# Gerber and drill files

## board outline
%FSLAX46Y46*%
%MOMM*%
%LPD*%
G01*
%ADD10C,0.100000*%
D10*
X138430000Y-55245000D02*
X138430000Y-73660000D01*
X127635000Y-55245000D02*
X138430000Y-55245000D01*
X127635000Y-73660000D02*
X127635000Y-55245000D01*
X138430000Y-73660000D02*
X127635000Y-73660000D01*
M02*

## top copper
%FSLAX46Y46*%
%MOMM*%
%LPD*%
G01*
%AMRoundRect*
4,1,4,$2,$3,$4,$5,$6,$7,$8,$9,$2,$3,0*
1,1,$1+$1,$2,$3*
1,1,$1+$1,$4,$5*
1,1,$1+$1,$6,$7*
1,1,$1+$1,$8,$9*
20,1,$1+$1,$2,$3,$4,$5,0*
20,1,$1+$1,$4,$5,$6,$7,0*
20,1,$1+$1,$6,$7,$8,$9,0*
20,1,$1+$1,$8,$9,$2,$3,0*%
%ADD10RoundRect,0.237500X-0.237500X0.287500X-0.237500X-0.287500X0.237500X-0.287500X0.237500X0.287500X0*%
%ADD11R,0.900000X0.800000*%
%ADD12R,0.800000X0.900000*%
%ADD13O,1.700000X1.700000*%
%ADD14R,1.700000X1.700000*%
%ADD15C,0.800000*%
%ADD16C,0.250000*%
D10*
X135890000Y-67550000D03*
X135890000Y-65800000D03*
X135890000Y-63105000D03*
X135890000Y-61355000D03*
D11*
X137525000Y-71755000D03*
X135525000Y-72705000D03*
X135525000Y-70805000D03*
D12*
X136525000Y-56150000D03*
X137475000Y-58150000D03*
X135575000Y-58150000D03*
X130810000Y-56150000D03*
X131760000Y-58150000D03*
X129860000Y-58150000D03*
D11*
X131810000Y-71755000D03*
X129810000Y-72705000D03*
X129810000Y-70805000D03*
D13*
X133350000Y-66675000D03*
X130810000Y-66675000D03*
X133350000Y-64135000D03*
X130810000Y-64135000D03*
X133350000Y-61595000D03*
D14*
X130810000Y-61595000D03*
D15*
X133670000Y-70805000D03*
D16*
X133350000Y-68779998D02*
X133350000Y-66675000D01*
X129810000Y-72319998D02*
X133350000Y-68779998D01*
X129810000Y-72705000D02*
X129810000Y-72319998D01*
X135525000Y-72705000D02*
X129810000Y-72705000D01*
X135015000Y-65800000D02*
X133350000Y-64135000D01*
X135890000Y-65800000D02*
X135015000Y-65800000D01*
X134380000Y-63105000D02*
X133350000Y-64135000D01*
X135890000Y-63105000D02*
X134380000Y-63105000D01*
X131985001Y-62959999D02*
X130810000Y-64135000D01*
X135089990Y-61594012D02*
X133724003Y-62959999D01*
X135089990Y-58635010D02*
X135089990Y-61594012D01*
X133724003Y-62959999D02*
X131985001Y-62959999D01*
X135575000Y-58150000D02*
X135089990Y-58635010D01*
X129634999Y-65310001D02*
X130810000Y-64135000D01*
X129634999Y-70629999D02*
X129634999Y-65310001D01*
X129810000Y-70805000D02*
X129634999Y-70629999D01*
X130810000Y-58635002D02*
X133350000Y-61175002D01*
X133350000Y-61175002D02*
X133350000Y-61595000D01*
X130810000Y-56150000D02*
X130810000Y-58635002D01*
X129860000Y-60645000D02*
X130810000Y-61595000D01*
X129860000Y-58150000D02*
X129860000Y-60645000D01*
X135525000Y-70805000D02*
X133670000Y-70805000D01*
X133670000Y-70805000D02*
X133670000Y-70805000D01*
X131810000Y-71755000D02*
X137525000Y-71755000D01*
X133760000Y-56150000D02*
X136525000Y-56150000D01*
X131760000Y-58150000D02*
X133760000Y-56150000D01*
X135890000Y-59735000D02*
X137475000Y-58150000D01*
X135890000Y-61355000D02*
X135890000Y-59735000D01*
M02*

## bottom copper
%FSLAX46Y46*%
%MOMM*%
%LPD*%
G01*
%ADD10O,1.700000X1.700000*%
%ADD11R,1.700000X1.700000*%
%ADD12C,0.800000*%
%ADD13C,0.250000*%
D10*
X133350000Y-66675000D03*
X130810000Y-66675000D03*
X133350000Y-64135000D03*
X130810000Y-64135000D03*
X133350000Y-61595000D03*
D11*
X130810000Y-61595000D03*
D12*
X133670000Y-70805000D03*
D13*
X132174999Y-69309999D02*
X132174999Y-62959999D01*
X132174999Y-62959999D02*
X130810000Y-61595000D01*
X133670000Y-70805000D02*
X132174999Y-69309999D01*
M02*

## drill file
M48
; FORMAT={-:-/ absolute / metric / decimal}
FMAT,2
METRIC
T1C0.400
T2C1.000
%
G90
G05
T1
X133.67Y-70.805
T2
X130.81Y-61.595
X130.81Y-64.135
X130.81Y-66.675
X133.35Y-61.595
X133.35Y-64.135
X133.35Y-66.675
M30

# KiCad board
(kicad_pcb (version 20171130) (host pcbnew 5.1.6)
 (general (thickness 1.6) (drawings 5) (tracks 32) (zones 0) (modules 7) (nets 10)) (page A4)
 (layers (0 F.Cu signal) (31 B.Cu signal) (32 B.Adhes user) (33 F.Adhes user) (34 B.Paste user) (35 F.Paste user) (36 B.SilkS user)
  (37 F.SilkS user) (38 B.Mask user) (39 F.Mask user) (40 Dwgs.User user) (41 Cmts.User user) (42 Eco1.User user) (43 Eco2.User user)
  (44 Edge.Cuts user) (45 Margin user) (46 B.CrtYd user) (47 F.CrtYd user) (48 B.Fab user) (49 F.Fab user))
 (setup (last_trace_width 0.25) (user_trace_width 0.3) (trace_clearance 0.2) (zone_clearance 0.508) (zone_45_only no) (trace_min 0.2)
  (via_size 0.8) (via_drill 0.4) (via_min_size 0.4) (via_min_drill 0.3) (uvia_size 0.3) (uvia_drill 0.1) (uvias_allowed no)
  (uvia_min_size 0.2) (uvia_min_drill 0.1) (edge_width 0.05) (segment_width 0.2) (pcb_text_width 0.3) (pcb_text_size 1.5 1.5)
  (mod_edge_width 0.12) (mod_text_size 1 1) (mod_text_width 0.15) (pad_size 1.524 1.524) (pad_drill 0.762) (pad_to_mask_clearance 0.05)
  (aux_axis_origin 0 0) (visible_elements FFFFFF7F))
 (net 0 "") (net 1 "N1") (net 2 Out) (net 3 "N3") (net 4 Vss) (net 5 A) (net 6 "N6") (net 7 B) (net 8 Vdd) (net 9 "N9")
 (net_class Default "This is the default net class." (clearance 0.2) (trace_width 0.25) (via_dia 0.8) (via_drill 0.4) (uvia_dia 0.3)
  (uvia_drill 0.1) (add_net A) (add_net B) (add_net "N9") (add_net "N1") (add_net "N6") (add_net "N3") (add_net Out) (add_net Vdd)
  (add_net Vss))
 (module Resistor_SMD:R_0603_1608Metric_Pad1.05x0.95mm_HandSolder (layer F.Cu) (at 135.89 66.675 270)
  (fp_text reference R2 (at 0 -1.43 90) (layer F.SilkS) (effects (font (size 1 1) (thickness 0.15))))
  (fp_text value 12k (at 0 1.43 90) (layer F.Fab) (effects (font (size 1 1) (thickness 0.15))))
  (pad 2 smd roundrect (at 0.875 0 270) (size 1.05 0.95) (layers F.Cu F.Paste F.Mask) (roundrect_rratio 0.25) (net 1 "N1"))
  (pad 1 smd roundrect (at -0.875 0 270) (size 1.05 0.95) (layers F.Cu F.Paste F.Mask) (roundrect_rratio 0.25) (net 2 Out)))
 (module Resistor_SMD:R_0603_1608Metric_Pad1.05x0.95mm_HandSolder (layer F.Cu) (at 135.89 62.23 270)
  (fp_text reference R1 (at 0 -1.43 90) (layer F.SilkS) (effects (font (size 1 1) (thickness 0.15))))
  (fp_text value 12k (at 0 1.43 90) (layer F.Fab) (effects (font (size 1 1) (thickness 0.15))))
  (pad 2 smd roundrect (at 0.875 0 270) (size 1.05 0.95) (layers F.Cu F.Paste F.Mask) (roundrect_rratio 0.25) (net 2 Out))
  (pad 1 smd roundrect (at -0.875 0 270) (size 1.05 0.95) (layers F.Cu F.Paste F.Mask) (roundrect_rratio 0.25) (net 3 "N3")))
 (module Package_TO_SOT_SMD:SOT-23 (layer F.Cu) (at 136.525 71.755)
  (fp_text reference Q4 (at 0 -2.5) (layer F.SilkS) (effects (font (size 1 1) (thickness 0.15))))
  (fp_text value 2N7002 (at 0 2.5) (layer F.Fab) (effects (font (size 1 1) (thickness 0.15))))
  (pad 3 smd rect (at 1 0) (size 0.9 0.8) (layers F.Cu F.Paste F.Mask) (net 1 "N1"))
  (pad 2 smd rect (at -1 0.95) (size 0.9 0.8) (layers F.Cu F.Paste F.Mask) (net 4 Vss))
  (pad 1 smd rect (at -1 -0.95) (size 0.9 0.8) (layers F.Cu F.Paste F.Mask) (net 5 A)))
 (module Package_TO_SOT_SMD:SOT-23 (layer F.Cu) (at 136.525 57.15 90)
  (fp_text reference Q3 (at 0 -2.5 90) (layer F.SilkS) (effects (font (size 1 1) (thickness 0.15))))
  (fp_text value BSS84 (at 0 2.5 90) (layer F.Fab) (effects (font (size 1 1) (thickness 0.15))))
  (pad 3 smd rect (at 1 0 90) (size 0.9 0.8) (layers F.Cu F.Paste F.Mask) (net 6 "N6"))
  (pad 2 smd rect (at -1 0.95 90) (size 0.9 0.8) (layers F.Cu F.Paste F.Mask) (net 3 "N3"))
  (pad 1 smd rect (at -1 -0.95 90) (size 0.9 0.8) (layers F.Cu F.Paste F.Mask) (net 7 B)))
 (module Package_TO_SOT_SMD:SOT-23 (layer F.Cu) (at 130.81 57.15 90)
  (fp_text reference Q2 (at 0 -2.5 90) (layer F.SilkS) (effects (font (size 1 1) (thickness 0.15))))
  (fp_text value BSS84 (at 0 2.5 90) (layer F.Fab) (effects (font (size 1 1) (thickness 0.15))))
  (pad 3 smd rect (at 1 0 90) (size 0.9 0.8) (layers F.Cu F.Paste F.Mask) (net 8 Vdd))
  (pad 2 smd rect (at -1 0.95 90) (size 0.9 0.8) (layers F.Cu F.Paste F.Mask) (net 6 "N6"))
  (pad 1 smd rect (at -1 -0.95 90) (size 0.9 0.8) (layers F.Cu F.Paste F.Mask) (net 5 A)))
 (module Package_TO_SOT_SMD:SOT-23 (layer F.Cu) (at 130.81 71.755)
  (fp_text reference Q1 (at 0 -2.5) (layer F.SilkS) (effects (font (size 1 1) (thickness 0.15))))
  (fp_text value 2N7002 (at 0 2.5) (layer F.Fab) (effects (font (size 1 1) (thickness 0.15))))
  (pad 3 smd rect (at 1 0) (size 0.9 0.8) (layers F.Cu F.Paste F.Mask) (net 1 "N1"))
  (pad 2 smd rect (at -1 0.95) (size 0.9 0.8) (layers F.Cu F.Paste F.Mask) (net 4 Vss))
  (pad 1 smd rect (at -1 -0.95) (size 0.9 0.8) (layers F.Cu F.Paste F.Mask) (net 7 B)))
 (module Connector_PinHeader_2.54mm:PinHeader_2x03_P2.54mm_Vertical (layer F.Cu) (at 130.81 61.595)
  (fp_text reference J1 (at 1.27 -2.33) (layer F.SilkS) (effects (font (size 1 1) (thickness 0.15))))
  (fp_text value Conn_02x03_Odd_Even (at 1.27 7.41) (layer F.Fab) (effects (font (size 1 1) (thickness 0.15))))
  (pad 6 thru_hole oval (at 2.54 5.08) (size 1.7 1.7) (drill 1) (layers *.Cu *.Mask) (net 4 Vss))
  (pad 5 thru_hole oval (at 0 5.08) (size 1.7 1.7) (drill 1) (layers *.Cu *.Mask) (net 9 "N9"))
  (pad 4 thru_hole oval (at 2.54 2.54) (size 1.7 1.7) (drill 1) (layers *.Cu *.Mask) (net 2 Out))
  (pad 3 thru_hole oval (at 0 2.54) (size 1.7 1.7) (drill 1) (layers *.Cu *.Mask) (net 7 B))
  (pad 2 thru_hole oval (at 2.54 0) (size 1.7 1.7) (drill 1) (layers *.Cu *.Mask) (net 8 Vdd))
  (pad 1 thru_hole rect (at 0 0) (size 1.7 1.7) (drill 1) (layers *.Cu *.Mask) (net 5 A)))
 (gr_line (start 138.43 55.245) (end 138.43 73.66) (layer Edge.Cuts) (width 0.1))
 (gr_line (start 127.635 55.245) (end 138.43 55.245) (layer Edge.Cuts) (width 0.1))
 (gr_line (start 127.635 73.66) (end 127.635 55.245) (layer Edge.Cuts) (width 0.1))
 (gr_line (start 138.43 73.66) (end 127.635 73.66) (layer Edge.Cuts) (width 0.1))
 (segment (start 133.35 68.779998) (end 133.35 66.675) (width 0.25) (layer F.Cu) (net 4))
 (segment (start 129.81 72.319998) (end 133.35 68.779998) (width 0.25) (layer F.Cu) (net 4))
 (segment (start 129.81 72.705) (end 129.81 72.319998) (width 0.25) (layer F.Cu) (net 4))
 (segment (start 135.525 72.705) (end 129.81 72.705) (width 0.25) (layer F.Cu) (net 4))
 (segment (start 135.015 65.8) (end 133.35 64.135) (width 0.25) (layer F.Cu) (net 2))
 (segment (start 135.89 65.8) (end 135.015 65.8) (width 0.25) (layer F.Cu) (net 2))
 (segment (start 134.38 63.105) (end 133.35 64.135) (width 0.25) (layer F.Cu) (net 2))
 (segment (start 135.89 63.105) (end 134.38 63.105) (width 0.25) (layer F.Cu) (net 2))
 (segment (start 131.985001 62.959999) (end 130.81 64.135) (width 0.25) (layer F.Cu) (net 7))
 (segment (start 135.08999 61.594012) (end 133.724003 62.959999) (width 0.25) (layer F.Cu) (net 7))
 (segment (start 135.08999 58.63501) (end 135.08999 61.594012) (width 0.25) (layer F.Cu) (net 7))
 (segment (start 133.724003 62.959999) (end 131.985001 62.959999) (width 0.25) (layer F.Cu) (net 7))
 (segment (start 135.575 58.15) (end 135.08999 58.63501) (width 0.25) (layer F.Cu) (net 7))
 (segment (start 129.634999 65.310001) (end 130.81 64.135) (width 0.25) (layer F.Cu) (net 7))
 (segment (start 129.634999 70.629999) (end 129.634999 65.310001) (width 0.25) (layer F.Cu) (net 7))
 (segment (start 129.81 70.805) (end 129.634999 70.629999) (width 0.25) (layer F.Cu) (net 7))
 (segment (start 130.81 58.635002) (end 133.35 61.175002) (width 0.25) (layer F.Cu) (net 8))
 (segment (start 133.35 61.175002) (end 133.35 61.595) (width 0.25) (layer F.Cu) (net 8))
 (segment (start 130.81 56.15) (end 130.81 58.635002) (width 0.25) (layer F.Cu) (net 8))
 (segment (start 129.86 60.645) (end 130.81 61.595) (width 0.25) (layer F.Cu) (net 5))
 (segment (start 129.86 58.15) (end 129.86 60.645) (width 0.25) (layer F.Cu) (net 5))
 (segment (start 135.525 70.805) (end 133.67 70.805) (width 0.25) (layer F.Cu) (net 5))
 (segment (start 133.67 70.805) (end 133.67 70.805) (width 0.25) (layer F.Cu) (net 5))
 (via (at 133.67 70.805) (size 0.8) (drill 0.4) (layers F.Cu B.Cu) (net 5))
 (segment (start 132.174999 69.309999) (end 132.174999 62.959999) (width 0.25) (layer B.Cu) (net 5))
 (segment (start 132.174999 62.959999) (end 130.81 61.595) (width 0.25) (layer B.Cu) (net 5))
 (segment (start 133.67 70.805) (end 132.174999 69.309999) (width 0.25) (layer B.Cu) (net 5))
 (segment (start 131.81 71.755) (end 137.525 71.755) (width 0.25) (layer F.Cu) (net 1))
 (segment (start 133.76 56.15) (end 136.525 56.15) (width 0.25) (layer F.Cu) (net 6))
 (segment (start 131.76 58.15) (end 133.76 56.15) (width 0.25) (layer F.Cu) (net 6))
 (segment (start 135.89 59.735) (end 137.475 58.15) (width 0.25) (layer F.Cu) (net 3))
 (segment (start 135.89 61.355) (end 135.89 59.735) (width 0.25) (layer F.Cu) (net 3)))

